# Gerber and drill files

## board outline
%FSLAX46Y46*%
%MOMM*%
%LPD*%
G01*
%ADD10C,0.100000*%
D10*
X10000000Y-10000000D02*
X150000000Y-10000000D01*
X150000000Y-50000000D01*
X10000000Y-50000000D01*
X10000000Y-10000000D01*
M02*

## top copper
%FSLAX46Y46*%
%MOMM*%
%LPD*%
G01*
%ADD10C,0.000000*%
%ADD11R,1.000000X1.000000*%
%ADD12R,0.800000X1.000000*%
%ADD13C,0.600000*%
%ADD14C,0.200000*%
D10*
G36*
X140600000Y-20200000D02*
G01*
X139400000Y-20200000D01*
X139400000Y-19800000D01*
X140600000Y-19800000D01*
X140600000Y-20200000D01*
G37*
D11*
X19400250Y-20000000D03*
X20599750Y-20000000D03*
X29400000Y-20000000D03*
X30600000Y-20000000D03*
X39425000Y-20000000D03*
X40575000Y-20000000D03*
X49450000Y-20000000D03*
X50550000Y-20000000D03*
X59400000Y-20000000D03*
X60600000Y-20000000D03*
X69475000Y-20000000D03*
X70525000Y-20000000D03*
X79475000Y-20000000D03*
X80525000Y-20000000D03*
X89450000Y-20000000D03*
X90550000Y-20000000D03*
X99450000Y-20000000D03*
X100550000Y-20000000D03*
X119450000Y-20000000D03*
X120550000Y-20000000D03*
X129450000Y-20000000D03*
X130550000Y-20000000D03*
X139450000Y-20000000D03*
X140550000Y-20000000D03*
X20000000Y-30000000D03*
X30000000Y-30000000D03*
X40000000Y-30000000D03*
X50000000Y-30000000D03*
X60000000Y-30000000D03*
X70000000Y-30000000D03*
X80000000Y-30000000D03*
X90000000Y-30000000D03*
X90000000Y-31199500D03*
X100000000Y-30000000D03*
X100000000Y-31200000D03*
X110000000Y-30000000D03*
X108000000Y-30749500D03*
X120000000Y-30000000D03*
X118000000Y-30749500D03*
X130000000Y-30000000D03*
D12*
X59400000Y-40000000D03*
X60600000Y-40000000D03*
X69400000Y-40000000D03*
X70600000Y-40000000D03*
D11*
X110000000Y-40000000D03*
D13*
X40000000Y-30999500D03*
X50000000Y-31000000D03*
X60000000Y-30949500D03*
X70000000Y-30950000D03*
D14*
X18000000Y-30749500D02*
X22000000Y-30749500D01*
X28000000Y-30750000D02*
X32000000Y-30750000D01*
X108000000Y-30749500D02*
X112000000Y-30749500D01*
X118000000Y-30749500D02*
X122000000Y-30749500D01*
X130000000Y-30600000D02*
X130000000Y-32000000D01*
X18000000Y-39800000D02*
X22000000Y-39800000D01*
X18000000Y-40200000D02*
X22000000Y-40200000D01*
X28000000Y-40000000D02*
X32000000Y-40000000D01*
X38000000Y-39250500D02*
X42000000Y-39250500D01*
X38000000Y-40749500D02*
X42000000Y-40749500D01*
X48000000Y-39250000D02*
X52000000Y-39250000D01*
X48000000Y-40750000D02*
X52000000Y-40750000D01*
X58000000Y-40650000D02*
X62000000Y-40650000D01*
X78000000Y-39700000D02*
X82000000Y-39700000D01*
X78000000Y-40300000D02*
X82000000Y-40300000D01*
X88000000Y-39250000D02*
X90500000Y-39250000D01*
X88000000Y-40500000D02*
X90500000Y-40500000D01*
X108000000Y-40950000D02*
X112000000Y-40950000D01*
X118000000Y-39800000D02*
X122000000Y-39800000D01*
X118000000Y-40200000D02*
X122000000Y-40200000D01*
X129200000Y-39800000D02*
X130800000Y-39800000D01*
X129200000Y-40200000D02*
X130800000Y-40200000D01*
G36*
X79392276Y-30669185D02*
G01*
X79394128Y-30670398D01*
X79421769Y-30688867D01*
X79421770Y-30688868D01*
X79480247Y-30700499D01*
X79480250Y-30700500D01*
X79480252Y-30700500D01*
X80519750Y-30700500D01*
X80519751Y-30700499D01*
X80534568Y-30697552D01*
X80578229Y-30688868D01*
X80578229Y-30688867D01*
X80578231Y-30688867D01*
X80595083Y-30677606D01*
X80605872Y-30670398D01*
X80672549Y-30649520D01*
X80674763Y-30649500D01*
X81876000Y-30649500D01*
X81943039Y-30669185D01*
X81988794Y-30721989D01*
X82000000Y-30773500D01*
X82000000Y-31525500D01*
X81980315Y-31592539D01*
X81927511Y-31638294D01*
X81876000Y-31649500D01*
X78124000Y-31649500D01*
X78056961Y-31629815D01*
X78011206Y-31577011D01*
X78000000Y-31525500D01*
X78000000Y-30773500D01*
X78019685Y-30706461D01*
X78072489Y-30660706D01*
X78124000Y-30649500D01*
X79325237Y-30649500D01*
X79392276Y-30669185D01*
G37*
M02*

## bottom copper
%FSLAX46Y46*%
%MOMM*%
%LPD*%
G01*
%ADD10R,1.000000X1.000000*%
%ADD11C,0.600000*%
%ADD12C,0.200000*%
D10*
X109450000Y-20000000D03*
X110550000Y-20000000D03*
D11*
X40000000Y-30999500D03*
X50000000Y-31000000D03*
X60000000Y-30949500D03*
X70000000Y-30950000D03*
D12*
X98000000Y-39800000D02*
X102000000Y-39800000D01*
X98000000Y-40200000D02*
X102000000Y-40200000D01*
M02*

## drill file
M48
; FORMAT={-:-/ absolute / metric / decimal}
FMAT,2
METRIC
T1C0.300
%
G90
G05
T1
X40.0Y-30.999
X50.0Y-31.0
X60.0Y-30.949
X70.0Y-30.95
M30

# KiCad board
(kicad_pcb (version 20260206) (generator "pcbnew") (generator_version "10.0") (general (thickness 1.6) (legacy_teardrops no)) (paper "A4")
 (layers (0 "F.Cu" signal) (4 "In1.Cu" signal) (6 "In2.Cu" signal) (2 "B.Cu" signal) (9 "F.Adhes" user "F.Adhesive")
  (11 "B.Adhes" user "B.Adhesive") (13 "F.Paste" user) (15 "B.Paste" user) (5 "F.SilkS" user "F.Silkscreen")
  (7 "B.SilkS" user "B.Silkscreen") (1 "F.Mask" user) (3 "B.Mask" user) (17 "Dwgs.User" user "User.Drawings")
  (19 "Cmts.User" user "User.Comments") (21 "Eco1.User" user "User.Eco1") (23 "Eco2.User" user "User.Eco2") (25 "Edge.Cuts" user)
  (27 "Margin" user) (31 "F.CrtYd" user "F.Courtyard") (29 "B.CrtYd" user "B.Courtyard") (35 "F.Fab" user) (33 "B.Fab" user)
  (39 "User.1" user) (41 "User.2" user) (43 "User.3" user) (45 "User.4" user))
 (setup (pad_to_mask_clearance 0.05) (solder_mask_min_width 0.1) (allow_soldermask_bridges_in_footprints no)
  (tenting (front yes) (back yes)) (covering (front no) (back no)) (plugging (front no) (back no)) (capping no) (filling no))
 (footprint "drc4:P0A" (layer "F.Cu") (at 19.40025 20)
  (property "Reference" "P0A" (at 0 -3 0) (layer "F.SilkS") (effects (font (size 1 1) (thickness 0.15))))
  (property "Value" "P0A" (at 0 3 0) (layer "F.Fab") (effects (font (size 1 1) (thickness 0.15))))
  (pad "1" smd rect (at 0 0) (size 1 1) (layers "F.Cu" "F.Mask" "F.Paste") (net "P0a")))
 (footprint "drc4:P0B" (layer "F.Cu") (at 20.59975 20)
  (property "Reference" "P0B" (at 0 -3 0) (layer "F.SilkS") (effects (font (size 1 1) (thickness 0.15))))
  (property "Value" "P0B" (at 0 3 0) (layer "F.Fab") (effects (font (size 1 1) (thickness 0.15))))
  (pad "1" smd rect (at 0 0) (size 1 1) (layers "F.Cu" "F.Mask" "F.Paste") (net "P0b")))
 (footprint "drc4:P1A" (layer "F.Cu") (at 29.4 20)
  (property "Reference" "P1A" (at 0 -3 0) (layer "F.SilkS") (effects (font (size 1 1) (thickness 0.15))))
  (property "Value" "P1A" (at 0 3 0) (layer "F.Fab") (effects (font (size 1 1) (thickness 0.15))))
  (pad "1" smd rect (at 0 0) (size 1 1) (layers "F.Cu" "F.Mask" "F.Paste") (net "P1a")))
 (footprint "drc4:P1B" (layer "F.Cu") (at 30.6 20)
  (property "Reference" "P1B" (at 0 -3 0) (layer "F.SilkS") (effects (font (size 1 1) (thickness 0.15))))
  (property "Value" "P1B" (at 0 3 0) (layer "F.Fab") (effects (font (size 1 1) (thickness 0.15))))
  (pad "1" smd rect (at 0 0) (size 1 1) (layers "F.Cu" "F.Mask" "F.Paste") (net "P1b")))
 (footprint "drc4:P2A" (layer "F.Cu") (at 39.425 20)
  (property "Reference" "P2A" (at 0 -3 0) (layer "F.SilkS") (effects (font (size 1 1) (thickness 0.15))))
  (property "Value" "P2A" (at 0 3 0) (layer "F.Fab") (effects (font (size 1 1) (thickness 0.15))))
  (pad "1" smd rect (at 0 0) (size 1 1) (layers "F.Cu" "F.Mask" "F.Paste") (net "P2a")))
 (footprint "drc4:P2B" (layer "F.Cu") (at 40.575 20)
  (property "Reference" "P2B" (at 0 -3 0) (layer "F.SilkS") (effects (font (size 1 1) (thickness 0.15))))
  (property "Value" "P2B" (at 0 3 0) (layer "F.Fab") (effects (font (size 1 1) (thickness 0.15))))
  (pad "1" smd rect (at 0 0) (size 1 1) (layers "F.Cu" "F.Mask" "F.Paste") (solder_mask_margin 0) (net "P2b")))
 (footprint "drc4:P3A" (layer "F.Cu") (at 49.45 20)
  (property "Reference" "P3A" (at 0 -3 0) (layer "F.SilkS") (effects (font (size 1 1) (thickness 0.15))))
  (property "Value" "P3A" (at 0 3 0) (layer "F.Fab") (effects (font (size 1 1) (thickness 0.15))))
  (pad "1" smd rect (at 0 0) (size 1 1) (layers "F.Cu" "F.Mask" "F.Paste") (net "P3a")))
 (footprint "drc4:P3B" (layer "F.Cu") (at 50.55 20)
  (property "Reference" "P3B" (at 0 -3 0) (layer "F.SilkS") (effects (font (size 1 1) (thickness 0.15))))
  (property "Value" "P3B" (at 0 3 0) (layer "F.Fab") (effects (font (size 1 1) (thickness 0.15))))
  (pad "1" smd rect (at 0 0) (size 1 1) (layers "F.Cu" "F.Mask" "F.Paste") (solder_mask_margin -0.05) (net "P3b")))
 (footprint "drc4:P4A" (layer "F.Cu") (at 59.4 20)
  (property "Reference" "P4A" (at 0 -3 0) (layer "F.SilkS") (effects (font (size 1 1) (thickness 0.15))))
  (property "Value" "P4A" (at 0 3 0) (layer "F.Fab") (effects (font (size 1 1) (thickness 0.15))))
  (pad "1" smd rect (at 0 0) (size 1 1) (layers "F.Cu" "F.Mask" "F.Paste") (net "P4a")))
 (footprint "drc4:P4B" (layer "F.Cu") (at 60.6 20)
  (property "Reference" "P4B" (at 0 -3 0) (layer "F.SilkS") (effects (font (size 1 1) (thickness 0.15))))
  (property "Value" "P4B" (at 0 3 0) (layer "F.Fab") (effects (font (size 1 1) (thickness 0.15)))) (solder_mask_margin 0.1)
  (pad "1" smd rect (at 0 0) (size 1 1) (layers "F.Cu" "F.Mask" "F.Paste") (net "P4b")))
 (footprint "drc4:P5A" (layer "F.Cu") (at 69.475 20)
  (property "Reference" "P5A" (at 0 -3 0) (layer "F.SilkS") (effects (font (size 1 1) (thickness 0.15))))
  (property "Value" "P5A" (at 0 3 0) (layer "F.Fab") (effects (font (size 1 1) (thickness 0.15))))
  (pad "1" smd rect (at 0 0) (size 1 1) (layers "F.Cu" "F.Mask" "F.Paste") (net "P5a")))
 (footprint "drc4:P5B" (layer "F.Cu") (at 70.525 20)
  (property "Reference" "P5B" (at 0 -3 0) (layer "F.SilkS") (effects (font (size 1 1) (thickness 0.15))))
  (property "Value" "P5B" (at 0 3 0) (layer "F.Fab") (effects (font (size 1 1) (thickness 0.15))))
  (pad "1" smd rect (at 0 0) (size 1 1) (layers "F.Cu" "F.Mask" "F.Paste") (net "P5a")))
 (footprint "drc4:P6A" (layer "F.Cu") (at 79.475 20)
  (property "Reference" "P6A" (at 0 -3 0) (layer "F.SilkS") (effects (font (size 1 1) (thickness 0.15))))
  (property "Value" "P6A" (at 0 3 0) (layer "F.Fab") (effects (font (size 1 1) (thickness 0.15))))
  (pad "1" smd rect (at 0 0) (size 1 1) (layers "F.Cu" "F.Mask" "F.Paste")))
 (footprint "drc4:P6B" (layer "F.Cu") (at 80.525 20)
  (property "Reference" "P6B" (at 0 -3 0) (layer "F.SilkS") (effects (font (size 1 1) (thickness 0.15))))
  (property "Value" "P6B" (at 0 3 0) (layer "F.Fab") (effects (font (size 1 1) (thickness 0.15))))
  (pad "1" smd rect (at 0 0) (size 1 1) (layers "F.Cu" "F.Mask" "F.Paste")))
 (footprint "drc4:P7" (layer "F.Cu") (at 90 20)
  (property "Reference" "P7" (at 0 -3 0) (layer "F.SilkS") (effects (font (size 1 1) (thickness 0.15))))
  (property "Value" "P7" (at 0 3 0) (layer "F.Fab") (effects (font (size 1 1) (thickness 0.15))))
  (pad "1" smd rect (at -0.55 0) (size 1 1) (layers "F.Cu" "F.Mask" "F.Paste") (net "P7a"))
  (pad "2" smd rect (at 0.55 0) (size 1 1) (layers "F.Cu" "F.Mask" "F.Paste") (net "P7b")))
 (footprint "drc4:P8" (layer "F.Cu") (at 100 20)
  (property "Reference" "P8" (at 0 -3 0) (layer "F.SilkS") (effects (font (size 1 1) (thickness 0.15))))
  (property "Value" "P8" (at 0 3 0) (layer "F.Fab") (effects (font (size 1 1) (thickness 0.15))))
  (pad "1" smd rect (at -0.55 0) (size 1 1) (layers "F.Cu" "F.Mask" "F.Paste") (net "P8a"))
  (pad "2" smd rect (at 0.55 0) (size 1 1) (layers "F.Cu" "F.Mask" "F.Paste") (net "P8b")))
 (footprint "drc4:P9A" (layer "B.Cu") (at 109.45 20)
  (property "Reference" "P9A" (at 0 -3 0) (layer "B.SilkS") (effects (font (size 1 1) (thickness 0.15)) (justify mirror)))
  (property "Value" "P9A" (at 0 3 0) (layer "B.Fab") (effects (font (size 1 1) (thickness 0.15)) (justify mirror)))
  (pad "1" smd rect (at 0 0) (size 1 1) (layers "B.Cu" "B.Mask" "B.Paste") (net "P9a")))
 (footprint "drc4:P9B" (layer "B.Cu") (at 110.55 20)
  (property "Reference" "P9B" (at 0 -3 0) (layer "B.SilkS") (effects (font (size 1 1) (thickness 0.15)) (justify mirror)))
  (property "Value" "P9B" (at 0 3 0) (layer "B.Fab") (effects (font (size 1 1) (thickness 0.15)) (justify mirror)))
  (pad "1" smd rect (at 0 0) (size 1 1) (layers "B.Cu" "B.Mask" "B.Paste") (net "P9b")))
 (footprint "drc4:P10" (layer "F.Cu") (at 120 20)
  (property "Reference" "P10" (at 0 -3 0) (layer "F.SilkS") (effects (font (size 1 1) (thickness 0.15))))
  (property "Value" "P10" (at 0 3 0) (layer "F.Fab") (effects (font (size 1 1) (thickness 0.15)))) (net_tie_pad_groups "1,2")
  (pad "1" smd rect (at -0.55 0) (size 1 1) (layers "F.Cu" "F.Mask" "F.Paste") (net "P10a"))
  (pad "2" smd rect (at 0.55 0) (size 1 1) (layers "F.Cu" "F.Mask" "F.Paste") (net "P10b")))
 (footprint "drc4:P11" (layer "F.Cu") (at 130 20)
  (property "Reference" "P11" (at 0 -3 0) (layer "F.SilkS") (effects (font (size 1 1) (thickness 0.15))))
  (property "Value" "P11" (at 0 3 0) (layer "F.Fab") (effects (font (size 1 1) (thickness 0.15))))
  (pad "1" smd rect (at -0.55 0) (size 1 1) (layers "F.Cu" "F.Mask" "F.Paste") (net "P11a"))
  (pad "1" smd rect (at 0.55 0) (size 1 1) (layers "F.Cu" "F.Mask" "F.Paste") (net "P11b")))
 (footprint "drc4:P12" (layer "F.Cu") (at 140 20)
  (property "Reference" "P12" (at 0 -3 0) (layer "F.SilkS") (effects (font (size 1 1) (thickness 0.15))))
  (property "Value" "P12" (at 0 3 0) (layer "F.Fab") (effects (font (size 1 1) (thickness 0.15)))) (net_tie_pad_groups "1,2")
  (fp_poly (pts (xy -0.6 -0.2) (xy 0.6 -0.2) (xy 0.6 0.2) (xy -0.6 0.2)) (stroke (width 0) (type solid)) (fill yes) (layer "F.Cu"))
  (pad "1" smd rect (at -0.55 0) (size 1 1) (layers "F.Cu" "F.Mask" "F.Paste") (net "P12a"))
  (pad "2" smd rect (at 0.55 0) (size 1 1) (layers "F.Cu" "F.Mask" "F.Paste") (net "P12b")))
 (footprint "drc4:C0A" (layer "F.Cu") (at 20 30)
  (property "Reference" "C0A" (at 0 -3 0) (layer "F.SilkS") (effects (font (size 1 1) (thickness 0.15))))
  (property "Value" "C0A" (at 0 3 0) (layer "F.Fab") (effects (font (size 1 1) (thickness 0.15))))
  (pad "1" smd rect (at 0 0) (size 1 1) (layers "F.Cu" "F.Mask" "F.Paste") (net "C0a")))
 (segment (start 18 30.7495) (end 22 30.7495) (width 0.2) (layer "F.Cu") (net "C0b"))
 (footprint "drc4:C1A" (layer "F.Cu") (at 30 30)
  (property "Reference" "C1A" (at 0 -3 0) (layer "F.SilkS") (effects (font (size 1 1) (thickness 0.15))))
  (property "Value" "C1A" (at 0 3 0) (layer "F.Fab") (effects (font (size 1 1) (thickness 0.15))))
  (pad "1" smd rect (at 0 0) (size 1 1) (layers "F.Cu" "F.Mask" "F.Paste") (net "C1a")))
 (segment (start 28 30.75) (end 32 30.75) (width 0.2) (layer "F.Cu") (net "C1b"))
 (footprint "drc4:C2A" (layer "F.Cu") (at 40 30)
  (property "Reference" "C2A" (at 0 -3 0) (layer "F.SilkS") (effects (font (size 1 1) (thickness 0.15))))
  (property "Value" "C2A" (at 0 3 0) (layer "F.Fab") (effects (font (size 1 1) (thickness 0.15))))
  (pad "1" smd rect (at 0 0) (size 1 1) (layers "F.Cu" "F.Mask" "F.Paste") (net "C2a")))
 (via (at 40 30.9995) (size 0.6) (drill 0.3) (layers "F.Cu" "B.Cu") (tenting (front no) (back no)) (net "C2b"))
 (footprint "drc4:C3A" (layer "F.Cu") (at 50 30)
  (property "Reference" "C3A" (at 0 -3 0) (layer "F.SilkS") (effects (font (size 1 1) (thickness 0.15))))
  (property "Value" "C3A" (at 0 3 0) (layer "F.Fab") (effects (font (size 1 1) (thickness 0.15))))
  (pad "1" smd rect (at 0 0) (size 1 1) (layers "F.Cu" "F.Mask" "F.Paste") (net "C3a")))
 (via (at 50 31) (size 0.6) (drill 0.3) (layers "F.Cu" "B.Cu") (tenting (front no) (back no)) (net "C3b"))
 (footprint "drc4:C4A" (layer "F.Cu") (at 60 30)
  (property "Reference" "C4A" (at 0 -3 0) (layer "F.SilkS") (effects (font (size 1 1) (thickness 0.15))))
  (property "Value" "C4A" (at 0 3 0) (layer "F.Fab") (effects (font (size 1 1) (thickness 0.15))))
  (pad "1" smd rect (at 0 0) (size 1 1) (layers "F.Cu" "F.Mask" "F.Paste") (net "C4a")))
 (via (at 60 30.9495) (size 0.6) (drill 0.3) (layers "F.Cu" "B.Cu") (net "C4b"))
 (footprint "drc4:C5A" (layer "F.Cu") (at 70 30)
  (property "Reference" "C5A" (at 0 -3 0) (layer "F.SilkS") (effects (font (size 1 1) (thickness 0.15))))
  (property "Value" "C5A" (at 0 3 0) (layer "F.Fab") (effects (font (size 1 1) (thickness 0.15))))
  (pad "1" smd rect (at 0 0) (size 1 1) (layers "F.Cu" "F.Mask" "F.Paste") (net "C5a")))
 (via (at 70 30.95) (size 0.6) (drill 0.3) (layers "F.Cu" "B.Cu") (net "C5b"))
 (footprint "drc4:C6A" (layer "F.Cu") (at 80 30)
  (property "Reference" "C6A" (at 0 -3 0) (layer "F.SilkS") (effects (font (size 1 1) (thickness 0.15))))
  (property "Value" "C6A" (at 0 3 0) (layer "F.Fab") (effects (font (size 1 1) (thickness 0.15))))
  (pad "1" smd rect (at 0 0) (size 1 1) (layers "F.Cu" "F.Mask" "F.Paste") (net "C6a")))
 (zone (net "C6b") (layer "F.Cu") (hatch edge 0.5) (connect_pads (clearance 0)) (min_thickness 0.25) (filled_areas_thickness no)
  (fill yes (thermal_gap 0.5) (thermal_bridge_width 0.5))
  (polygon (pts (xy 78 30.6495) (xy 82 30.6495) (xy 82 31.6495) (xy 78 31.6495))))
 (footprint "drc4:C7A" (layer "F.Cu") (at 90 30)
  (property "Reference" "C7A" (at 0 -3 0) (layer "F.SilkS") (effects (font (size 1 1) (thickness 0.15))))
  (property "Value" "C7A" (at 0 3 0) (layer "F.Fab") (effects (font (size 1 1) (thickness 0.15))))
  (pad "1" smd rect (at 0 0) (size 1 1) (layers "F.Cu" "F.Mask" "F.Paste") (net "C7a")))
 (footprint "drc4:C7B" (layer "F.Cu") (at 90 31.1995)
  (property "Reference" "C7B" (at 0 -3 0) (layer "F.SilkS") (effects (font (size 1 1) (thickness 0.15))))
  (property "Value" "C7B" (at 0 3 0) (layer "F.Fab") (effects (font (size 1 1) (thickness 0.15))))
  (pad "1" smd rect (at 0 0) (size 1 1) (layers "F.Cu") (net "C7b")))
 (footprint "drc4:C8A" (layer "F.Cu") (at 100 30)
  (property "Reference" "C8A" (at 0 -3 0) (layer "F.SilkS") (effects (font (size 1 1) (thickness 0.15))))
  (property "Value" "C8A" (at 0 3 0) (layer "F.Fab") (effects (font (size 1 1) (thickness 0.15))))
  (pad "1" smd rect (at 0 0) (size 1 1) (layers "F.Cu" "F.Mask" "F.Paste") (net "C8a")))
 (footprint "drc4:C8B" (layer "F.Cu") (at 100 31.2)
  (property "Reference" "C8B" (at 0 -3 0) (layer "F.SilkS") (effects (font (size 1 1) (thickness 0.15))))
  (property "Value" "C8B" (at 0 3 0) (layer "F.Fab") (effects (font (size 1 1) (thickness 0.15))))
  (pad "1" smd rect (at 0 0) (size 1 1) (layers "F.Cu") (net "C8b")))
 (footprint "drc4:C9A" (layer "F.Cu") (at 110 30)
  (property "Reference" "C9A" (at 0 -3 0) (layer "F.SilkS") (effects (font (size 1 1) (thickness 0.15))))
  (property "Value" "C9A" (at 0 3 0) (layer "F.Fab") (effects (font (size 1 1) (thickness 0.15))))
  (pad "1" smd rect (at 0 0) (size 1 1) (layers "F.Cu" "F.Mask" "F.Paste") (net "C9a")))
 (segment (start 108 30.7495) (end 112 30.7495) (width 0.2) (layer "F.Cu") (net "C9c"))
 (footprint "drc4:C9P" (layer "F.Cu") (at 108 30.7495)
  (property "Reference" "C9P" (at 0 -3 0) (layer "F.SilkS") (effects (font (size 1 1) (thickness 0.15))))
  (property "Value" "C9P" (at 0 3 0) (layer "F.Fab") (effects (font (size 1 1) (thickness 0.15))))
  (pad "1" smd rect (at 0 0) (size 1 1) (layers "F.Cu" "F.Mask" "F.Paste") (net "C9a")))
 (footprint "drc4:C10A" (layer "F.Cu") (at 120 30)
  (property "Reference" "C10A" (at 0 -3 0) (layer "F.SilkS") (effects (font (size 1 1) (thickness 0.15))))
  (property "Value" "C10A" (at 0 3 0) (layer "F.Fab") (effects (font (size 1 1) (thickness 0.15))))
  (pad "1" smd rect (at 0 0) (size 1 1) (layers "F.Cu" "F.Mask" "F.Paste") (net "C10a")))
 (segment (start 118 30.7495) (end 122 30.7495) (width 0.2) (layer "F.Cu") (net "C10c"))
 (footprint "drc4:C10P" (layer "F.Cu") (at 118 30.7495)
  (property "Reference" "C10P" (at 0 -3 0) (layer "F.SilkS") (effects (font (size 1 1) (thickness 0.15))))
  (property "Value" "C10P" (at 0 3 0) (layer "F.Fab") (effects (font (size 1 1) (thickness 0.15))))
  (pad "1" smd rect (at 0 0) (size 1 1) (layers "F.Cu" "F.Mask" "F.Paste") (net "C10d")))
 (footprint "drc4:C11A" (layer "F.Cu") (at 130 30)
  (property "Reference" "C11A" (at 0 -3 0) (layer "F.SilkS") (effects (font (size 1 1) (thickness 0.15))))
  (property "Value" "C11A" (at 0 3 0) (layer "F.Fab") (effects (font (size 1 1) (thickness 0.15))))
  (pad "1" smd rect (at 0 0) (size 1 1) (layers "F.Cu" "F.Mask" "F.Paste") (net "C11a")))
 (segment (start 130 30.6) (end 130 32) (width 0.2) (layer "F.Cu") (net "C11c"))
 (segment (start 18 39.8) (end 22 39.8) (width 0.2) (layer "F.Cu") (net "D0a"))
 (segment (start 18 40.2) (end 22 40.2) (width 0.2) (layer "F.Cu") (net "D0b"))
 (segment (start 28 40) (end 32 40) (width 0.2) (layer "F.Cu") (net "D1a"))
 (segment (start 38 39.2505) (end 42 39.2505) (width 0.2) (layer "F.Cu") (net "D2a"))
 (segment (start 38 40.7495) (end 42 40.7495) (width 0.2) (layer "F.Cu") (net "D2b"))
 (segment (start 48 39.25) (end 52 39.25) (width 0.2) (layer "F.Cu") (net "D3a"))
 (segment (start 48 40.75) (end 52 40.75) (width 0.2) (layer "F.Cu") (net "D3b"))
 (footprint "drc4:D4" (layer "F.Cu") (at 60 40)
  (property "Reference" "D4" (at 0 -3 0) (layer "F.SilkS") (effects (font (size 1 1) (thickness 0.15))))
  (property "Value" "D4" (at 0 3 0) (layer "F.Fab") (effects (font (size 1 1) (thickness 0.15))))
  (pad "1" smd rect (at -0.6 0) (size 0.8 1) (layers "F.Cu" "F.Mask" "F.Paste") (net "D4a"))
  (pad "2" smd rect (at 0.6 0) (size 0.8 1) (layers "F.Cu" "F.Mask" "F.Paste") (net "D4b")))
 (segment (start 58 40.65) (end 62 40.65) (width 0.2) (layer "F.Cu") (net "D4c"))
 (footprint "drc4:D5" (layer "F.Cu") (at 70 40)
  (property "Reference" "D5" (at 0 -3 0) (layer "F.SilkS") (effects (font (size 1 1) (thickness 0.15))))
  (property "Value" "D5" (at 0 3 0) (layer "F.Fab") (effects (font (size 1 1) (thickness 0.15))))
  (pad "1" smd rect (at -0.6 0) (size 0.8 1) (layers "F.Cu" "F.Mask" "F.Paste") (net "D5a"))
  (pad "2" smd rect (at 0.6 0) (size 0.8 1) (layers "F.Cu" "F.Mask" "F.Paste") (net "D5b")))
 (segment (start 78 39.7) (end 82 39.7) (width 0.2) (layer "F.Cu") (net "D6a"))
 (segment (start 78 40.3) (end 82 40.3) (width 0.2) (layer "F.Cu") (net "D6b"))
 (segment (start 88 39.25) (end 90.5 39.25) (width 0.2) (layer "F.Cu") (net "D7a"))
 (segment (start 88 40.5) (end 90.5 40.5) (width 0.2) (layer "F.Cu") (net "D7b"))
 (segment (start 98 39.8) (end 102 39.8) (width 0.2) (layer "B.Cu") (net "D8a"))
 (segment (start 98 40.2) (end 102 40.2) (width 0.2) (layer "B.Cu") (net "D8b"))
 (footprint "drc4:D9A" (layer "F.Cu") (at 110 40)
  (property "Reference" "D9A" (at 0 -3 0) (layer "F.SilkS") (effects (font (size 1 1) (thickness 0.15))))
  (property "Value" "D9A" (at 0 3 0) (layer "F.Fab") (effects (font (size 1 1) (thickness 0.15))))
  (pad "1" smd rect (at 0 0) (size 1 1) (layers "F.Cu" "F.Mask" "F.Paste") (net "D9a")))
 (segment (start 108 40.95) (end 112 40.95) (width 0.2) (layer "F.Cu") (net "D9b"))
 (segment (start 118 39.8) (end 122 39.8) (width 0.2) (layer "F.Cu") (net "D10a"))
 (segment (start 118 40.2) (end 122 40.2) (width 0.2) (layer "F.Cu") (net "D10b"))
 (segment (start 129.2 39.8) (end 130.8 39.8) (width 0.2) (layer "F.Cu") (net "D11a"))
 (segment (start 129.2 40.2) (end 130.8 40.2) (width 0.2) (layer "F.Cu") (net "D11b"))
 (gr_rect (start 10 10) (end 150 50) (stroke (width 0.1) (type solid)) (fill no) (layer "Edge.Cuts")))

